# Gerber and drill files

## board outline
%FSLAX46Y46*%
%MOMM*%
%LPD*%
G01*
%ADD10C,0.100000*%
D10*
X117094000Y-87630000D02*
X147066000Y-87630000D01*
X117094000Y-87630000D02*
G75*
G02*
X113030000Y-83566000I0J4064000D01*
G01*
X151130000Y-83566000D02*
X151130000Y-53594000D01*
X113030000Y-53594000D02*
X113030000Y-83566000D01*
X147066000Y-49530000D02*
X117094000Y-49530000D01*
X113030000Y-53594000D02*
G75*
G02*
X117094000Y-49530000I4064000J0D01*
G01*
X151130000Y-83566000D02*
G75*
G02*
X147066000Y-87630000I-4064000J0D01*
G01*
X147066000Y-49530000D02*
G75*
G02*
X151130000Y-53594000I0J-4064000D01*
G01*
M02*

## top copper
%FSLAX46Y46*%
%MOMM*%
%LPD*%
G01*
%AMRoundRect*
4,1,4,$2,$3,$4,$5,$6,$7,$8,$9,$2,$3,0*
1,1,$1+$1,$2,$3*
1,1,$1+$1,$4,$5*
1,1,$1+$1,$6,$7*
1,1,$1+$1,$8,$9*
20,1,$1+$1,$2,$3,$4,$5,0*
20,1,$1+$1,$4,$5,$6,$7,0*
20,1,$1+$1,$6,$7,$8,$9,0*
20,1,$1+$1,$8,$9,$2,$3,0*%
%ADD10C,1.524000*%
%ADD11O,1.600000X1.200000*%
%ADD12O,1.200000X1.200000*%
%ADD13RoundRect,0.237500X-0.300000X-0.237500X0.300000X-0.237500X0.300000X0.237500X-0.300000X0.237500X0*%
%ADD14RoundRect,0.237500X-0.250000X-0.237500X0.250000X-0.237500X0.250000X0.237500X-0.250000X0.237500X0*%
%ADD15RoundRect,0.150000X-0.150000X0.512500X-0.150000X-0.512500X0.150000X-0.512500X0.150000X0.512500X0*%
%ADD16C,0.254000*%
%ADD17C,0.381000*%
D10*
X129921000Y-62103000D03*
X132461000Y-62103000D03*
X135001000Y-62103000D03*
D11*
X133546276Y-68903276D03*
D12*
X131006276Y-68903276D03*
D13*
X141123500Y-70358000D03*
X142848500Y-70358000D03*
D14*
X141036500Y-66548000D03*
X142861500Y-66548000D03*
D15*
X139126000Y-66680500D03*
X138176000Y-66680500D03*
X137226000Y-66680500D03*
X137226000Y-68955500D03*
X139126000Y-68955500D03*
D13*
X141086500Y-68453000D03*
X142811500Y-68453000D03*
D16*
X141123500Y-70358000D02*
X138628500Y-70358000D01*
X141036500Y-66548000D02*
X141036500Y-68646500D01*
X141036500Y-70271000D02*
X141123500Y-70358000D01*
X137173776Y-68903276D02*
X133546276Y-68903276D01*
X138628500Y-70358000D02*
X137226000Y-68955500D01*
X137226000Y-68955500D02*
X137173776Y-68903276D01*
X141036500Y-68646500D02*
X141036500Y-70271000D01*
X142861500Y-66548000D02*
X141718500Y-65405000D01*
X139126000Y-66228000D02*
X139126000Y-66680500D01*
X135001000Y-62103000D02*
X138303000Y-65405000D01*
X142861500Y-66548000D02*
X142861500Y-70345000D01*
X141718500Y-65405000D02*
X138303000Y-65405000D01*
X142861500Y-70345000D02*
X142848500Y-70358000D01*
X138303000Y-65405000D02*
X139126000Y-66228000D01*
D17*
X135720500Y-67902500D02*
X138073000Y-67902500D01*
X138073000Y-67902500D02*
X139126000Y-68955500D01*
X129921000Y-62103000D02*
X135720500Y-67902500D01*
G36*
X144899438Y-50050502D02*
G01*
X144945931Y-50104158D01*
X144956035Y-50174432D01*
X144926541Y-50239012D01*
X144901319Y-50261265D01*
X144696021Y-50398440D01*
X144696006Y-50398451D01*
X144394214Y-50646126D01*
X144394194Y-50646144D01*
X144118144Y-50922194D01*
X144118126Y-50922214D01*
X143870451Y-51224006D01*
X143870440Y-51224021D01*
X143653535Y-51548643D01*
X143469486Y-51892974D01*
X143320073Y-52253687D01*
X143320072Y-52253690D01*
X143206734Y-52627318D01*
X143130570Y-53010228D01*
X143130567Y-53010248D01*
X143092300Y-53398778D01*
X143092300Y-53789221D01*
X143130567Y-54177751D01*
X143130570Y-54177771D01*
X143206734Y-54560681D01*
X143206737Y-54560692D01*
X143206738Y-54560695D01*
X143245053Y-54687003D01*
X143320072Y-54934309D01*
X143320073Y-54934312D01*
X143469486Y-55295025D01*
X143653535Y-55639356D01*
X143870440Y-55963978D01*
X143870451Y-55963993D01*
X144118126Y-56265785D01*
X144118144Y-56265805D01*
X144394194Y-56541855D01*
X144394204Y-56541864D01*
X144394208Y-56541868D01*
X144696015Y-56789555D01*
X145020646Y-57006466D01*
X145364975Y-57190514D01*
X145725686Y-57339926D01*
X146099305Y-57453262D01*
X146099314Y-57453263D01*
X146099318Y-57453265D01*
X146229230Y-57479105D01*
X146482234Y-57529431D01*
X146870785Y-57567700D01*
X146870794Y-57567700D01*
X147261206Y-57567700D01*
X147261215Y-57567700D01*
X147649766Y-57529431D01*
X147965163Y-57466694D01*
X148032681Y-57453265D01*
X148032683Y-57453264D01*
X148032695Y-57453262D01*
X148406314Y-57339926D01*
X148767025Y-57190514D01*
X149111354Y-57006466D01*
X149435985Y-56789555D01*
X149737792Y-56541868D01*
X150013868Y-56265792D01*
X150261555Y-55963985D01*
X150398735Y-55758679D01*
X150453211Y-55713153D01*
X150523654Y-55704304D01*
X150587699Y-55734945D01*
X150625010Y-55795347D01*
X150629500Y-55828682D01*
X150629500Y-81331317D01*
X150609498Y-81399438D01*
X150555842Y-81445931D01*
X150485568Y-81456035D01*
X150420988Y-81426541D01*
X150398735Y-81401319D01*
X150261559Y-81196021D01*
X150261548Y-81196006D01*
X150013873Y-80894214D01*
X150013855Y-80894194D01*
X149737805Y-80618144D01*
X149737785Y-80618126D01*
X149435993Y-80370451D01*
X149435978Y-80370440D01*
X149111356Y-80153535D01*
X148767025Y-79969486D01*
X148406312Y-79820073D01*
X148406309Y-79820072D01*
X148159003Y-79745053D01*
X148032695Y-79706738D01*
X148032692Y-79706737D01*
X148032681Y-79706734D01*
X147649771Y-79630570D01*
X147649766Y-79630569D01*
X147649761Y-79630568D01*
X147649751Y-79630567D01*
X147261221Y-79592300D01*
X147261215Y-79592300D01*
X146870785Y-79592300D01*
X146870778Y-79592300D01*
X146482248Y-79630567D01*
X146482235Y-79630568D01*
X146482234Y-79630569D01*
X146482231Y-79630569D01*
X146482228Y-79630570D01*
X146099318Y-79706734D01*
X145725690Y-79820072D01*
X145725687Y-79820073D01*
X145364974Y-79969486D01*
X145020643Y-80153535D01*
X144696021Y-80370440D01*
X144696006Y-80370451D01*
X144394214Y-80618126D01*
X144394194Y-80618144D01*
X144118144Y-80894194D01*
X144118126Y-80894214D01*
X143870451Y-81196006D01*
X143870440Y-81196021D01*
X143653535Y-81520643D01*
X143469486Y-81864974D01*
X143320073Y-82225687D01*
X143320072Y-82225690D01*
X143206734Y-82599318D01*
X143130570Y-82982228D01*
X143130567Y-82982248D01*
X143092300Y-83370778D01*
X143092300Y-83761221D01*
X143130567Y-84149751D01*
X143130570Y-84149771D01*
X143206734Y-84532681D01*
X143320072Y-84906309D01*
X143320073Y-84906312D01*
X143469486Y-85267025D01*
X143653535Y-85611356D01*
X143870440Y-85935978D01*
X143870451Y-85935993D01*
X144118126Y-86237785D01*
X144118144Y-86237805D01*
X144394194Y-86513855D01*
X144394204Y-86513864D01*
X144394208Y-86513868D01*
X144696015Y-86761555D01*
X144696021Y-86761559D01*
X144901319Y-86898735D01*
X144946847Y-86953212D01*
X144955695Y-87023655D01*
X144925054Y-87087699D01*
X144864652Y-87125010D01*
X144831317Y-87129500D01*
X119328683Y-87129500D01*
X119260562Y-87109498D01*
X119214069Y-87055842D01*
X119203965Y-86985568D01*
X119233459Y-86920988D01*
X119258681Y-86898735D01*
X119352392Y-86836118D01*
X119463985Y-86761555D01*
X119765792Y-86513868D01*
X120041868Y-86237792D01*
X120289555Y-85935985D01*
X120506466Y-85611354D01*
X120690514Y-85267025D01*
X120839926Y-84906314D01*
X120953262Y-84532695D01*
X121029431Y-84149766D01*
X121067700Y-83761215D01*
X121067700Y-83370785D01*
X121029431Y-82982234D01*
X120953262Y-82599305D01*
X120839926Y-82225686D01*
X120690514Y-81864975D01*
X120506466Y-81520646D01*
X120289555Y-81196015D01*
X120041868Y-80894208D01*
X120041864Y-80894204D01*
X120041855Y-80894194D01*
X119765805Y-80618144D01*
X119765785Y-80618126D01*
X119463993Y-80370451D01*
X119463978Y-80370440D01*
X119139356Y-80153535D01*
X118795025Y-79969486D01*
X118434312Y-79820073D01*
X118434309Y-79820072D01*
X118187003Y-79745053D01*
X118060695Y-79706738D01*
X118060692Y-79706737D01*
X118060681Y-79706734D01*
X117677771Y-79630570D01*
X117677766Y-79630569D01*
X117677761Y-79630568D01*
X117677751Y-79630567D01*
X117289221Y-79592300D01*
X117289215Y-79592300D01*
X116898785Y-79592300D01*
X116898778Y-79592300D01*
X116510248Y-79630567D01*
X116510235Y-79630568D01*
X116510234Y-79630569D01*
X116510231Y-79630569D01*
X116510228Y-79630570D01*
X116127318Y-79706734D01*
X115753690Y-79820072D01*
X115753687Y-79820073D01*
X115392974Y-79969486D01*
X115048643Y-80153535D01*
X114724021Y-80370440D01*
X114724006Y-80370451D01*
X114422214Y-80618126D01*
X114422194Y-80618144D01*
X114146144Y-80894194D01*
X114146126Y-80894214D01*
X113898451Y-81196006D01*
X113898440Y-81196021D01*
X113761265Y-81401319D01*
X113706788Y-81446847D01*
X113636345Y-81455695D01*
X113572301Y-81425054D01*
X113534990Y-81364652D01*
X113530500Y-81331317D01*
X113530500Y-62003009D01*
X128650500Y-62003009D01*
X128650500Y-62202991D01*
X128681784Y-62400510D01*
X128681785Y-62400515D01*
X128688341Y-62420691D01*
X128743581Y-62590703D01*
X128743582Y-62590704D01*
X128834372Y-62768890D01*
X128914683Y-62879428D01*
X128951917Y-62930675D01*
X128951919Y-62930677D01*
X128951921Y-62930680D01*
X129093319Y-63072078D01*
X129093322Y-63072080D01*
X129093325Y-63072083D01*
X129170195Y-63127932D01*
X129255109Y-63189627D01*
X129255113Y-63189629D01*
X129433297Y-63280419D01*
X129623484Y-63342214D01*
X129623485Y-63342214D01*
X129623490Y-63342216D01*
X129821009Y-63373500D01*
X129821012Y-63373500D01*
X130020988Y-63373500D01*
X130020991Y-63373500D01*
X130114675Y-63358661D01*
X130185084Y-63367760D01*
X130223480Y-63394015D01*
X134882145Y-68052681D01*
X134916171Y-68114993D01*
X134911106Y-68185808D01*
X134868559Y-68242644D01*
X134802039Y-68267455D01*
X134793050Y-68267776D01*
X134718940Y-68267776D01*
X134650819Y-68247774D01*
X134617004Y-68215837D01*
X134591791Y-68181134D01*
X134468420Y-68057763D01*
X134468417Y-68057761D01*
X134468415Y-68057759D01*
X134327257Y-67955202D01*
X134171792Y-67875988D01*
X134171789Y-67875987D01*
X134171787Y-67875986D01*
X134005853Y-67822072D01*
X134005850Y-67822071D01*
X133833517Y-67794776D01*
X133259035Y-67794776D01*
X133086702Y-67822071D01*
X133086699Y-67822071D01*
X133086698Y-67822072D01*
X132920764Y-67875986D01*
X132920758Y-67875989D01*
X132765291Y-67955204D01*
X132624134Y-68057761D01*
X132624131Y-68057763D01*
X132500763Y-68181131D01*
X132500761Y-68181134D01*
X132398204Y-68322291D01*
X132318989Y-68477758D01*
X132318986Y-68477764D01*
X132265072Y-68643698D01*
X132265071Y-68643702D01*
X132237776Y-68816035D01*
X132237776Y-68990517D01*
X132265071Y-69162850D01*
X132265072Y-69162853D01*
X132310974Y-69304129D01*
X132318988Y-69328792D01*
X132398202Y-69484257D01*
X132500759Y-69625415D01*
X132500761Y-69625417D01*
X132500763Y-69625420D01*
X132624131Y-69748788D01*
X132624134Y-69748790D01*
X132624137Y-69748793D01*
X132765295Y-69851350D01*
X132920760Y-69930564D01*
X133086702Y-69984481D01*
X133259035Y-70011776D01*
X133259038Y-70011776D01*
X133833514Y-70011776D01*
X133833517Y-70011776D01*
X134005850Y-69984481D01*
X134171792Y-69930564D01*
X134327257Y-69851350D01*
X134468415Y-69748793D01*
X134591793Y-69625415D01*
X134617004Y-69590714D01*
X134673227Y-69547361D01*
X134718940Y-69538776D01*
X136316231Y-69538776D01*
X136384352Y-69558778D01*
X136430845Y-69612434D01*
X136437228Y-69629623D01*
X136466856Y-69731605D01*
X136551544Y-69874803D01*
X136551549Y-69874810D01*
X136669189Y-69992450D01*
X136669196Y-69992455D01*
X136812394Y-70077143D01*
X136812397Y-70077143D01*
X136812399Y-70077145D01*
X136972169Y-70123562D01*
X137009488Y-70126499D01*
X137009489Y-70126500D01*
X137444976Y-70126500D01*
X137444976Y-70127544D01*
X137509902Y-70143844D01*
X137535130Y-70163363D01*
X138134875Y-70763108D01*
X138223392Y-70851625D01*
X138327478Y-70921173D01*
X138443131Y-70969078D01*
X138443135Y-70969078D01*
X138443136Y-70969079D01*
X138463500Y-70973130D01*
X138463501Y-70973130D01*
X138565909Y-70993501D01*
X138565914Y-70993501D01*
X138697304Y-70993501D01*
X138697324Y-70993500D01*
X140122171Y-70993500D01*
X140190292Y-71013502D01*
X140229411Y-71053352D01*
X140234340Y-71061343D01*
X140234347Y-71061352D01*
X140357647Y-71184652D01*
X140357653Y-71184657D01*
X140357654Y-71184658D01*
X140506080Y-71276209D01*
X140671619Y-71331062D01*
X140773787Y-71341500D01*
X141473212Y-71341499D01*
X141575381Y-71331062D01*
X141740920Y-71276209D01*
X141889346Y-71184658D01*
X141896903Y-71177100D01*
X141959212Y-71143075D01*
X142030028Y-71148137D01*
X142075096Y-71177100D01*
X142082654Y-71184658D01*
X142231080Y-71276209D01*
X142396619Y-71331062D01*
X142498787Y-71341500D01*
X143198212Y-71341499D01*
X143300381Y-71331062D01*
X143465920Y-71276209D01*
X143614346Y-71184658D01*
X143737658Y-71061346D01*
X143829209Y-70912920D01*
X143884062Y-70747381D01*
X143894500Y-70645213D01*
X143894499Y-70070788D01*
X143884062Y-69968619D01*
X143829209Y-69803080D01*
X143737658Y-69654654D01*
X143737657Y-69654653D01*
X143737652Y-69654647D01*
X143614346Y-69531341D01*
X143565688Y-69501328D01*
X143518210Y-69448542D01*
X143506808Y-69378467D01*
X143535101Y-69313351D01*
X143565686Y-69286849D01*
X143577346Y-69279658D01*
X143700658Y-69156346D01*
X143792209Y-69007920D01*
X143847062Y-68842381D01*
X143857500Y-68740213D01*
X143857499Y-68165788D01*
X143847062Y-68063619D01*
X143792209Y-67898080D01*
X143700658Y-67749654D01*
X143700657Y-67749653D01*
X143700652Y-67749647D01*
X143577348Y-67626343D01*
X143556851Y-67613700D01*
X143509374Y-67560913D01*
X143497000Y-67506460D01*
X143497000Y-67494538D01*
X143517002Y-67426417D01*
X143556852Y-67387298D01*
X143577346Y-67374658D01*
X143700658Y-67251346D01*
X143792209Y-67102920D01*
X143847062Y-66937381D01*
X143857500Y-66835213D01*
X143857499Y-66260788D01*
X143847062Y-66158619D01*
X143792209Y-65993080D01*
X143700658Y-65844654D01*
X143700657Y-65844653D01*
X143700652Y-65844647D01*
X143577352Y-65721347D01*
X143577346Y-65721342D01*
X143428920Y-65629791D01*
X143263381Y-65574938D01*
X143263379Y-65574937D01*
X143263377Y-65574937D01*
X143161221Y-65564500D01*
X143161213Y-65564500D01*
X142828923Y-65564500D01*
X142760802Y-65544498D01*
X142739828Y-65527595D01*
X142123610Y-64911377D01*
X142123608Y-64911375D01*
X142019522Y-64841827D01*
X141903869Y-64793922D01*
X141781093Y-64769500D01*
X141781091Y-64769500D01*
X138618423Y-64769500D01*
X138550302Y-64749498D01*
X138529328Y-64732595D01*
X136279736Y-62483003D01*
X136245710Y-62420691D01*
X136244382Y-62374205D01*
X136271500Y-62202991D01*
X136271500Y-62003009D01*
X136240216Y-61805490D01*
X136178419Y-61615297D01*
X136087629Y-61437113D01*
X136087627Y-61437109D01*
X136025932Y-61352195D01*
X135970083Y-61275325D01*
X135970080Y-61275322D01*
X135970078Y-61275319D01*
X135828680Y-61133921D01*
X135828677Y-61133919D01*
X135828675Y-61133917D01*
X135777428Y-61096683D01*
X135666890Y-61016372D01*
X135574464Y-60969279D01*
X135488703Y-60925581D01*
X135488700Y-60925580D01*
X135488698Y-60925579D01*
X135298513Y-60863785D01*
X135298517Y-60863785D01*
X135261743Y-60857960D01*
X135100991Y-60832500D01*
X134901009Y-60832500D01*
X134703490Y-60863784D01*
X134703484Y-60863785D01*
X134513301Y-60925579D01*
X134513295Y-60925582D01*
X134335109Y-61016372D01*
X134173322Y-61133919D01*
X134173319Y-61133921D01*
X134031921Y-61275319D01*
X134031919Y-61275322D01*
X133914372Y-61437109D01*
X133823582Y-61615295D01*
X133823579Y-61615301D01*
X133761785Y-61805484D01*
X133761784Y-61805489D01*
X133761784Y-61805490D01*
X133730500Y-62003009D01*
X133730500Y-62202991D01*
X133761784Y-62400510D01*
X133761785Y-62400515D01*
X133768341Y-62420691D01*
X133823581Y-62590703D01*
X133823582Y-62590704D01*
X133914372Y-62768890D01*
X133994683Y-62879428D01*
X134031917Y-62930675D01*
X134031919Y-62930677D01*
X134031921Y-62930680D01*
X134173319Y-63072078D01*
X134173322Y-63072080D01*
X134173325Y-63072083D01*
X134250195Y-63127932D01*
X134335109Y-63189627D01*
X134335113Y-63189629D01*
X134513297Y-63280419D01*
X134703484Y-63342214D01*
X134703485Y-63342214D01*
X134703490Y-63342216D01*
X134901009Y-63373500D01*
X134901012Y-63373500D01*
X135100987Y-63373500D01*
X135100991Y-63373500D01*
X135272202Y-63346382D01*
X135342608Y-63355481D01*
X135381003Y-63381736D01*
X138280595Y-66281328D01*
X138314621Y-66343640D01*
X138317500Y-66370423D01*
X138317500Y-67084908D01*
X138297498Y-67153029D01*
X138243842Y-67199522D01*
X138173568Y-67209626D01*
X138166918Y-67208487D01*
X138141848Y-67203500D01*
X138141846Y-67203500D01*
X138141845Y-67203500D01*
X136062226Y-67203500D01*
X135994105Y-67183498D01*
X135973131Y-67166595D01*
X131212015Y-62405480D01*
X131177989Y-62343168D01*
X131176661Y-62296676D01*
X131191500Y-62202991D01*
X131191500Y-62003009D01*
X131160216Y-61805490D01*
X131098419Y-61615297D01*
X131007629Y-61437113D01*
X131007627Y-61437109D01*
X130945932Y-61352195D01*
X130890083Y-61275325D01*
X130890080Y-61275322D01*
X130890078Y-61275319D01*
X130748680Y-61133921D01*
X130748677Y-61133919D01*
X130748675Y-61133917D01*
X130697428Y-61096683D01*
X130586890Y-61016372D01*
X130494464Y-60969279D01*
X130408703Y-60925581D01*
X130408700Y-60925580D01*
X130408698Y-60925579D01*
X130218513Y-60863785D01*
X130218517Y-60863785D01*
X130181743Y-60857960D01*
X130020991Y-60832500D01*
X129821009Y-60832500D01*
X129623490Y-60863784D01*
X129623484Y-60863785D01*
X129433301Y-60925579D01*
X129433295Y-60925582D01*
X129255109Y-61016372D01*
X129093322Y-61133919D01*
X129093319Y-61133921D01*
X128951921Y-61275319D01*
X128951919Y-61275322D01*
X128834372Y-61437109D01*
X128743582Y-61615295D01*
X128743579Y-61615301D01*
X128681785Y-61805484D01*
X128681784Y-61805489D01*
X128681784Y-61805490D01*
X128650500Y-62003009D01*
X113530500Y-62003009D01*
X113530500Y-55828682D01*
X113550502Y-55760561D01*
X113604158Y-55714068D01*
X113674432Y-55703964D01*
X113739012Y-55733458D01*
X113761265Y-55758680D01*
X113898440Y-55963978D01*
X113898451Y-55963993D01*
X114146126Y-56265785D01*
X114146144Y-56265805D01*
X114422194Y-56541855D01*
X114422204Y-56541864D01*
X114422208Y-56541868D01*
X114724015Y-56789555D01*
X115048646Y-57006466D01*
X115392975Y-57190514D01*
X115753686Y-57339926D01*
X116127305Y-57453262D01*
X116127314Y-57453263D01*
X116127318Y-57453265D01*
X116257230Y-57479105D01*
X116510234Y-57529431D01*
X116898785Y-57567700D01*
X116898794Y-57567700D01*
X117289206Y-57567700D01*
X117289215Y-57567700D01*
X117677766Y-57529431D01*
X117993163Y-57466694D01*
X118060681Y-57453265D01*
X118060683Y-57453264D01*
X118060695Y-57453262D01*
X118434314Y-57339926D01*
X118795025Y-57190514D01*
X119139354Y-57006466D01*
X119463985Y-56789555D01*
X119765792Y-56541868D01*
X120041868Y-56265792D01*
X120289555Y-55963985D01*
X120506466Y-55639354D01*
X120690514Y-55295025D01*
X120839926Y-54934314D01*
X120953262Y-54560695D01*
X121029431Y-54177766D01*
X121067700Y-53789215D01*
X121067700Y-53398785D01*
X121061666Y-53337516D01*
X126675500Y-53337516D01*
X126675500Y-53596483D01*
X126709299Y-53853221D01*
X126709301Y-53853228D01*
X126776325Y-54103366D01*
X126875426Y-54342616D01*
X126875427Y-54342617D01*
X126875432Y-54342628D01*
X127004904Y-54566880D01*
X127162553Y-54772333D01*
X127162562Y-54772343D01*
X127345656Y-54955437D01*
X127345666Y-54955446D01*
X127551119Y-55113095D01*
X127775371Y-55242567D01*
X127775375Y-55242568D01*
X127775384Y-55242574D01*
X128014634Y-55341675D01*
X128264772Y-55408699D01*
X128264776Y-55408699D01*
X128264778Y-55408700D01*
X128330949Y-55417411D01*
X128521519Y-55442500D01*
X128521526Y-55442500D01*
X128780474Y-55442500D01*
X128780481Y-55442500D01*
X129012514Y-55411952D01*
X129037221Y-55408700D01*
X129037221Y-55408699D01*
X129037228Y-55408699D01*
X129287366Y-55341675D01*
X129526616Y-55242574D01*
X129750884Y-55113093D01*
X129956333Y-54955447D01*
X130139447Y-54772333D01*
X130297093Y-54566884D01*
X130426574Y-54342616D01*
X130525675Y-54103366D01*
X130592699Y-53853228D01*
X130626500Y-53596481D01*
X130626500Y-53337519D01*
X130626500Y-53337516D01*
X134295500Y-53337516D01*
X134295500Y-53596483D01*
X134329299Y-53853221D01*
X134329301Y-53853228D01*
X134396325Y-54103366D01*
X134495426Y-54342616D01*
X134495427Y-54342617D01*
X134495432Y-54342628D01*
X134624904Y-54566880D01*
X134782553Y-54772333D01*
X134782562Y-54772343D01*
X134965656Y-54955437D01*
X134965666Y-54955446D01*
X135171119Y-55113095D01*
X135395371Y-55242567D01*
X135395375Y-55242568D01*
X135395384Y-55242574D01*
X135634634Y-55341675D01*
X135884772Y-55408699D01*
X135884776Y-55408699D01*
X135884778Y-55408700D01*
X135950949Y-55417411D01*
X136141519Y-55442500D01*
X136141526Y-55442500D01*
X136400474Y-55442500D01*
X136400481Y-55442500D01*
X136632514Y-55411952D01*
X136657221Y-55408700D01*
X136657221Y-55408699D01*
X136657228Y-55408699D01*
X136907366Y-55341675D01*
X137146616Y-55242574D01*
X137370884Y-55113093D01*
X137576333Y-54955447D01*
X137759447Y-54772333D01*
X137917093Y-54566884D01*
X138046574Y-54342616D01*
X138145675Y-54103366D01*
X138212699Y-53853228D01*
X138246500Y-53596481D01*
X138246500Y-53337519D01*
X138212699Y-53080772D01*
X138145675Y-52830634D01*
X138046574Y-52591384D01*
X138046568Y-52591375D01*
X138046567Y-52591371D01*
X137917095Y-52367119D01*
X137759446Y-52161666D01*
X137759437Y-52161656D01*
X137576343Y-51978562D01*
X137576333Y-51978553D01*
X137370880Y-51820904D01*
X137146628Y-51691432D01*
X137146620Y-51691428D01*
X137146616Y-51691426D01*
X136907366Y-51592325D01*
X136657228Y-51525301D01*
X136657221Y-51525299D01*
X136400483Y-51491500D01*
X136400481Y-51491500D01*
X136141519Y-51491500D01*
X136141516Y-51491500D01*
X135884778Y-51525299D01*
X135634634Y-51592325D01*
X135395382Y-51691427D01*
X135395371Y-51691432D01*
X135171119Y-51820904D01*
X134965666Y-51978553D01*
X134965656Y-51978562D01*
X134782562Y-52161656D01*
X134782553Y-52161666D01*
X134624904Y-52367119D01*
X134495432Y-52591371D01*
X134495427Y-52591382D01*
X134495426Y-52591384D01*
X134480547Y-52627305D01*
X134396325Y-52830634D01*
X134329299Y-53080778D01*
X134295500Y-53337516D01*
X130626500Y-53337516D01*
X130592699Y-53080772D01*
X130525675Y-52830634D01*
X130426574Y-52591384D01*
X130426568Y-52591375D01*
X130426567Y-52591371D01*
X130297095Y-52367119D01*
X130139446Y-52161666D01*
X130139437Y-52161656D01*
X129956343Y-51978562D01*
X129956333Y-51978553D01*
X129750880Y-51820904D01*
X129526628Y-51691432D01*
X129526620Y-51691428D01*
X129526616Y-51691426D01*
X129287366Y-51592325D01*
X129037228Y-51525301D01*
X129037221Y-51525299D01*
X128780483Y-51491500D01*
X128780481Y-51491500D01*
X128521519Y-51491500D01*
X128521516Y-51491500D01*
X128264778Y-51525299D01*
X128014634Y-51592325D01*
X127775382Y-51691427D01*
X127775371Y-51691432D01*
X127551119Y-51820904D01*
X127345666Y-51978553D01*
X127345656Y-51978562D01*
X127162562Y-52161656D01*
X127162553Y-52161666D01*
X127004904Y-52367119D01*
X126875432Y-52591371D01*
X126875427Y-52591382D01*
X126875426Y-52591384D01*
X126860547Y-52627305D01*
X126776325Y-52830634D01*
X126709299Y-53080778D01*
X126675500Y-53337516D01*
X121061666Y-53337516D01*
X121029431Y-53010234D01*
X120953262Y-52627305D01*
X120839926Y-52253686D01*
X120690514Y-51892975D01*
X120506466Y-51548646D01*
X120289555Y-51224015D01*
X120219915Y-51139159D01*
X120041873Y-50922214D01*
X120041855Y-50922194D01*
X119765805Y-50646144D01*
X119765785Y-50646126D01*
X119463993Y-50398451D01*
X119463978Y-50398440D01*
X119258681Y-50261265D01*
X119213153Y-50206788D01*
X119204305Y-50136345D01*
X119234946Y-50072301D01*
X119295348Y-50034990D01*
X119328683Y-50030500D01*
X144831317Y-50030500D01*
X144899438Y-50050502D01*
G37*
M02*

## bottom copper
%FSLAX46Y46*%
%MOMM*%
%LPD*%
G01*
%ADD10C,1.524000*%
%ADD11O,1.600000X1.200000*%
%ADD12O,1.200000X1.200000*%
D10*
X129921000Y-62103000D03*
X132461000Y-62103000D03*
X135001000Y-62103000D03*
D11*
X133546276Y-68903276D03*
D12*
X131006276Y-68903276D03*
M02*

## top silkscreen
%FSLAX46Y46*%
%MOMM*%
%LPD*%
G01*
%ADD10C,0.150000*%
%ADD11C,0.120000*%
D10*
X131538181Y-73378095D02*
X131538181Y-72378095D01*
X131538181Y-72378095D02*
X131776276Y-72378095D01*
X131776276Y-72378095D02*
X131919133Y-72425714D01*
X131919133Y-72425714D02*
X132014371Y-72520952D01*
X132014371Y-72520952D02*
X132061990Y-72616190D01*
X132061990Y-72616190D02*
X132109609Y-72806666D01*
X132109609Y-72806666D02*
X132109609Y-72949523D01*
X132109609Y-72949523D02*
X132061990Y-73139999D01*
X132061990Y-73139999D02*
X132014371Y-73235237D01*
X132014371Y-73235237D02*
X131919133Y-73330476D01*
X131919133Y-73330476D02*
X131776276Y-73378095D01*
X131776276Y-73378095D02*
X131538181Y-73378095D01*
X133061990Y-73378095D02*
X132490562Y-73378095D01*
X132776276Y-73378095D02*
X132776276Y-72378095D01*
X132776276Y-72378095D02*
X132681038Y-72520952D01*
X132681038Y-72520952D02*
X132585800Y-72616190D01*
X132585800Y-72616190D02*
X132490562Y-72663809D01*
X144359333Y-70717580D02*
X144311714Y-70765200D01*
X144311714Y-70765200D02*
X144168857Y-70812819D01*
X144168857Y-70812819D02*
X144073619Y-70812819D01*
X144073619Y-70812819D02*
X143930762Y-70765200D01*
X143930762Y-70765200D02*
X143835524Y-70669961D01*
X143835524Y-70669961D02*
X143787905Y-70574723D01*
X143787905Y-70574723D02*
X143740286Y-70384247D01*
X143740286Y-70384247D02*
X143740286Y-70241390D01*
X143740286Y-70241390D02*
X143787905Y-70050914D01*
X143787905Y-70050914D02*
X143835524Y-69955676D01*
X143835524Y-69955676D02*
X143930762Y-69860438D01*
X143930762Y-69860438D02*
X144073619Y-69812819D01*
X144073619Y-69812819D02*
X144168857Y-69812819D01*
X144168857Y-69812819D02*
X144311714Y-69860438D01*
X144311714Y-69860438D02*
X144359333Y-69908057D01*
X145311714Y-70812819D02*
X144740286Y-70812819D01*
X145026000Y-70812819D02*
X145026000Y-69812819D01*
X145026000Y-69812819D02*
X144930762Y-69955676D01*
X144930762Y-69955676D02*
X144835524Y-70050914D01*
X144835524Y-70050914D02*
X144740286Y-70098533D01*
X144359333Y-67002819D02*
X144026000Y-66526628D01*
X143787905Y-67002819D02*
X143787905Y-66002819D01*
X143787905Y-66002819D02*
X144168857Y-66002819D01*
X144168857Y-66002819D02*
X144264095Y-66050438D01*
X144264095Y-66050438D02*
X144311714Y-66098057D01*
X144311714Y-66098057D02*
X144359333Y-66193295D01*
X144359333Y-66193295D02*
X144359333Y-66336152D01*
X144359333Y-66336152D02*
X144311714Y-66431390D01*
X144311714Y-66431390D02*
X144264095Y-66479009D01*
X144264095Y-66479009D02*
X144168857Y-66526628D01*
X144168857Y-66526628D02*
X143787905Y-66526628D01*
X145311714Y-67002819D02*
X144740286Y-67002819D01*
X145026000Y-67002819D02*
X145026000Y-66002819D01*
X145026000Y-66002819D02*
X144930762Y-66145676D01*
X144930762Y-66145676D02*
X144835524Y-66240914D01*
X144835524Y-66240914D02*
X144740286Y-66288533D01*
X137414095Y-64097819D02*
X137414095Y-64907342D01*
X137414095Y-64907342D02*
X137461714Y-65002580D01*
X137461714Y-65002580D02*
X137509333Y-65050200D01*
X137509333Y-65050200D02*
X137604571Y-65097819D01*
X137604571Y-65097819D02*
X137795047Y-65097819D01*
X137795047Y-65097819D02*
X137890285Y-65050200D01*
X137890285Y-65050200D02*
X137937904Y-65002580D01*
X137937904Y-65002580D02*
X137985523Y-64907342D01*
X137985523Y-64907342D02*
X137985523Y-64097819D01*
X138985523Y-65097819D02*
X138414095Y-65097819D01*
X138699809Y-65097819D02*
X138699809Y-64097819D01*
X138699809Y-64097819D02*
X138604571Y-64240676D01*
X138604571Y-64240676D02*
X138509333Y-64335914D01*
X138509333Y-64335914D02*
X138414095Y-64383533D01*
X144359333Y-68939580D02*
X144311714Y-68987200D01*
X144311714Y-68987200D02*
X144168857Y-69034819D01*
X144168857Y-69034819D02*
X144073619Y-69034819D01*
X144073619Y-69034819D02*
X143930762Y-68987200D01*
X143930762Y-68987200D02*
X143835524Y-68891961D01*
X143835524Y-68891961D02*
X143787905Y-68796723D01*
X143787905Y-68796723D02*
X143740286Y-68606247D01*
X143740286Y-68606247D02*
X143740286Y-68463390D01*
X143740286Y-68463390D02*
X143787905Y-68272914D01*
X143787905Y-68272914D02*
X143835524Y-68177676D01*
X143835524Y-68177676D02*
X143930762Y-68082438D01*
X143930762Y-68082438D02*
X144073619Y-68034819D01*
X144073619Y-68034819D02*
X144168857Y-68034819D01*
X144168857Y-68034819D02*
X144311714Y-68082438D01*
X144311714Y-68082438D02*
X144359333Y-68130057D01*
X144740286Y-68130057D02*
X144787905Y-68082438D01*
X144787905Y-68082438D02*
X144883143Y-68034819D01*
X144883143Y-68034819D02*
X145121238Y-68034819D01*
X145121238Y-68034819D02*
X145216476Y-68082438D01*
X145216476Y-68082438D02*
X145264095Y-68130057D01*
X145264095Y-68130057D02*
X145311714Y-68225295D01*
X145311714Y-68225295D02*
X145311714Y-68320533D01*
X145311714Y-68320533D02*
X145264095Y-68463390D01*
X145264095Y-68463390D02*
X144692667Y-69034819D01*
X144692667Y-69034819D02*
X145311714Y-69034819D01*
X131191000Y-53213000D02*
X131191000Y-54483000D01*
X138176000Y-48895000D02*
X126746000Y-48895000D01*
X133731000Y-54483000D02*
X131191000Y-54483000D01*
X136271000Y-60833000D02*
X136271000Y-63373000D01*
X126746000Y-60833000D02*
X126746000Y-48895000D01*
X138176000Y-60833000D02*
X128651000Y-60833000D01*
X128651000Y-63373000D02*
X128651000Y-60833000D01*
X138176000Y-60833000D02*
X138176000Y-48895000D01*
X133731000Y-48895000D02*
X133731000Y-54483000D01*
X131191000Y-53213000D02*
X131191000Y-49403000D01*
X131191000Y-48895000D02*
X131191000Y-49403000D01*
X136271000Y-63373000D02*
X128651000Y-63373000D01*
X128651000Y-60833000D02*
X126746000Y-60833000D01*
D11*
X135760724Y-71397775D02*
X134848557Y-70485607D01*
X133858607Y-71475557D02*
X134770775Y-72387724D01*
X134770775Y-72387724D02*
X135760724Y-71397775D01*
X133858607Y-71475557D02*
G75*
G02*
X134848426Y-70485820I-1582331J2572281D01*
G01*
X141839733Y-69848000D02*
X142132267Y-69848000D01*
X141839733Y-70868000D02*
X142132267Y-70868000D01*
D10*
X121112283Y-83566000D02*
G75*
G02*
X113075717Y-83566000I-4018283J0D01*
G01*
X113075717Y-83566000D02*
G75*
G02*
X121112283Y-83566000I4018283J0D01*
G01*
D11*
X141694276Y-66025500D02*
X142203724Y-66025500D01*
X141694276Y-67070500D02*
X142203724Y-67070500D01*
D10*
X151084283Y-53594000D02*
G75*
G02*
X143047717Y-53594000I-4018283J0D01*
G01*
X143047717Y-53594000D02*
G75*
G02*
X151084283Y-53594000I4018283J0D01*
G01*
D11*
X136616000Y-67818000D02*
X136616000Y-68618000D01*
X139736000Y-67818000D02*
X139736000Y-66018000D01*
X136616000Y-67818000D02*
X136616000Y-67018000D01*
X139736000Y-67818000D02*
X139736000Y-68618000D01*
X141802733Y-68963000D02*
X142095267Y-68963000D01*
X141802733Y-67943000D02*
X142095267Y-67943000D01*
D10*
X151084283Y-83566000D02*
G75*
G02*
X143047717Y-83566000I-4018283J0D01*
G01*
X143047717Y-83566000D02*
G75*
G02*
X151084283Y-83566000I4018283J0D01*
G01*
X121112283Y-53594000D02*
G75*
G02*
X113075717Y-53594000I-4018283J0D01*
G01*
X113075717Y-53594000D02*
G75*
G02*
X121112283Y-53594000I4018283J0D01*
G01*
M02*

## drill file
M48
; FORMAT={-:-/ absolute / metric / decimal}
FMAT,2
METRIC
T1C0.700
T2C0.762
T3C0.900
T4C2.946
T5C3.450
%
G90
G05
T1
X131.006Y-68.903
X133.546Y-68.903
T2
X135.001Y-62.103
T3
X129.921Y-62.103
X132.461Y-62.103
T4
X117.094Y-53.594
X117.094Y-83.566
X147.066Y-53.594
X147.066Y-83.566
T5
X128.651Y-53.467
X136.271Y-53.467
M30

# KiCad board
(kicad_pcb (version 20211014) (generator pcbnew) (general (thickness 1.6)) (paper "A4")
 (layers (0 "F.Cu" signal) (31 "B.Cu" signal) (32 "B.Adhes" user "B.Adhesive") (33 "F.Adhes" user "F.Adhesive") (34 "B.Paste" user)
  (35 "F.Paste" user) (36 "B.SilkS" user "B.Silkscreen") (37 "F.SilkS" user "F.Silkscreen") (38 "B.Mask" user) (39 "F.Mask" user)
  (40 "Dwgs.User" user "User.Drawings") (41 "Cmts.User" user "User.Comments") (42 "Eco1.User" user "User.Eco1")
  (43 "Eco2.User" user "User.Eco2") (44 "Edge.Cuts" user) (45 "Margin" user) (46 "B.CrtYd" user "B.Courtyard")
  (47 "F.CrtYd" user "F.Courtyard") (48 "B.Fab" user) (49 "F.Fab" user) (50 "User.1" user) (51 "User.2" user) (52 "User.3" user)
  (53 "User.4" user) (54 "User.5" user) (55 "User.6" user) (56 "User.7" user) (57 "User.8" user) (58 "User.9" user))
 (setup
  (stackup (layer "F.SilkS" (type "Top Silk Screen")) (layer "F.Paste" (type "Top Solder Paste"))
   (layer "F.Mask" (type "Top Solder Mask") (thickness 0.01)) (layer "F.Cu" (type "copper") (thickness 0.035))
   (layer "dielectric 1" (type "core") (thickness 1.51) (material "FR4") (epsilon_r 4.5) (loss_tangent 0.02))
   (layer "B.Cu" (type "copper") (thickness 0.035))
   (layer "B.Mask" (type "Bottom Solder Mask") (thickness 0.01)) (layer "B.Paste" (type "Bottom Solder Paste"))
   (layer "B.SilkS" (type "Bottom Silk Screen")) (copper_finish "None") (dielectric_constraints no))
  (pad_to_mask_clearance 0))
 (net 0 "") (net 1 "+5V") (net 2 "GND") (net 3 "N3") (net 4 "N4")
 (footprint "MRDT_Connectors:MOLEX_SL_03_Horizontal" (layer "F.Cu") (at 129.921 62.103)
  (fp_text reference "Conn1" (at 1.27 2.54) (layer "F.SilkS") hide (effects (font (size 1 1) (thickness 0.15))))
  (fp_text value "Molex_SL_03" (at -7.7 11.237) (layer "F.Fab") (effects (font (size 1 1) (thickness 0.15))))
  (fp_line (start 1.27 -8.89) (end 1.27 -7.62) (layer "F.SilkS") (width 0.15))
  (fp_line (start 8.255 -13.208) (end -3.175 -13.208) (layer "F.SilkS") (width 0.15))
  (fp_line (start 3.81 -7.62) (end 1.27 -7.62) (layer "F.SilkS") (width 0.15))
  (fp_line (start 6.35 -1.27) (end 6.35 1.27) (layer "F.SilkS") (width 0.15))
  (fp_line (start -3.175 -1.27) (end -3.175 -13.208) (layer "F.SilkS") (width 0.15))
  (fp_line (start 8.255 -1.27) (end -1.27 -1.27) (layer "F.SilkS") (width 0.15))
  (fp_line (start -1.27 1.27) (end -1.27 -1.27) (layer "F.SilkS") (width 0.15))
  (fp_line (start 8.255 -1.27) (end 8.255 -13.208) (layer "F.SilkS") (width 0.15))
  (fp_line (start 3.81 -13.208) (end 3.81 -7.62) (layer "F.SilkS") (width 0.15))
  (fp_line (start 1.27 -8.89) (end 1.27 -12.7) (layer "F.SilkS") (width 0.15))
  (fp_line (start 1.27 -13.208) (end 1.27 -12.7) (layer "F.SilkS") (width 0.15))
  (fp_line (start 6.35 1.27) (end -1.27 1.27) (layer "F.SilkS") (width 0.15))
  (fp_line (start -1.27 -1.27) (end -3.175 -1.27) (layer "F.SilkS") (width 0.15))
  (pad "" np_thru_hole circle locked (at 6.35 -8.636) (size 3.45 3.45) (drill 3.45) (layers *.Cu *.Mask))
  (pad "" np_thru_hole circle locked (at -1.27 -8.636) (size 3.45 3.45) (drill 3.45) (layers *.Cu *.Mask))
  (pad "1" thru_hole circle locked (at 0 0) (size 1.524 1.524) (drill 0.9) (layers *.Cu *.Mask) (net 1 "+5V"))
  (pad "2" thru_hole circle locked (at 2.54 0) (size 1.524 1.524) (drill 0.9) (layers *.Cu *.Mask) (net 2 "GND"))
  (pad "3" thru_hole circle locked (at 5.08 0) (size 1.524 1.524) (drill 0.762) (layers *.Cu *.Mask) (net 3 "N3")))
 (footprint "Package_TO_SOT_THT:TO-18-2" (layer "F.Cu") (at 133.546276 68.903276 180)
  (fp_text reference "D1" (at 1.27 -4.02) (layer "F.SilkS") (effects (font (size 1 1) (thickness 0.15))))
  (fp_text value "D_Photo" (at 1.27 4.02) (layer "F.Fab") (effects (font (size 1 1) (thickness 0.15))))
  (fp_line (start -2.214448 -2.494499) (end -1.302281 -1.582331) (layer "F.SilkS") (width 0.12))
  (fp_line (start -0.312331 -2.572281) (end -1.224499 -3.484448) (layer "F.SilkS") (width 0.12))
  (fp_line (start -1.224499 -3.484448) (end -2.214448 -2.494499) (layer "F.SilkS") (width 0.12))
  (fp_arc (start -0.312331 -2.572281) (mid 3.405374 2.135551) (end -1.30215 -1.582544) (layer "F.SilkS") (width 0.12))
  (pad "1" thru_hole oval (at 0 0 180) (size 1.6 1.2) (drill 0.7) (layers *.Cu *.Mask) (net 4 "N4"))
  (pad "2" thru_hole oval (at 2.54 0 180) (size 1.2 1.2) (drill 0.7) (layers *.Cu *.Mask) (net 2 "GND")))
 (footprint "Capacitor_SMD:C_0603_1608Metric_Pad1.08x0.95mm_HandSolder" (layer "F.Cu") (at 141.986 70.358)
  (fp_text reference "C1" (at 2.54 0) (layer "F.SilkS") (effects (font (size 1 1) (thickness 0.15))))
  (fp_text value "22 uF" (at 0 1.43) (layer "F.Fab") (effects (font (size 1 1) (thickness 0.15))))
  (fp_line (start -0.146267 -0.51) (end 0.146267 -0.51) (layer "F.SilkS") (width 0.12))
  (fp_line (start -0.146267 0.51) (end 0.146267 0.51) (layer "F.SilkS") (width 0.12))
  (pad "1" smd roundrect (at -0.8625 0) (size 1.075 0.95) (layers "F.Cu" "F.Paste" "F.Mask") (roundrect_rratio 0.25) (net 4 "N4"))
  (pad "2" smd roundrect (at 0.8625 0) (size 1.075 0.95) (layers "F.Cu" "F.Paste" "F.Mask") (roundrect_rratio 0.25) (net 3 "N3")))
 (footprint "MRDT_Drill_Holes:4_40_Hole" (layer "F.Cu") (at 117.094 83.566) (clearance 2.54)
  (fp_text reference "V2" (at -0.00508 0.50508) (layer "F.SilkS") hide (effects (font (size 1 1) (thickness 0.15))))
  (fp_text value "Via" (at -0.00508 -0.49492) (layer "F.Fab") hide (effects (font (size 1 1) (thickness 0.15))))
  (fp_circle (center 0 0) (end -0.00508 4.01828) (layer "F.SilkS") (width 0.15) (fill none))
  (pad "" np_thru_hole circle locked (at 0 0) (size 2.9464 2.9464) (drill 2.9464) (layers *.Cu *.Mask) (clearance 2.5)))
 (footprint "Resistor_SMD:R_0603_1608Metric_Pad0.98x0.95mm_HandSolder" (layer "F.Cu") (at 141.949 66.548)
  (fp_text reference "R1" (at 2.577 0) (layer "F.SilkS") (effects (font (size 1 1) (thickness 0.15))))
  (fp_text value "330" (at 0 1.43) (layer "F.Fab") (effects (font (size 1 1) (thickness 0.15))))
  (fp_line (start -0.254724 -0.5225) (end 0.254724 -0.5225) (layer "F.SilkS") (width 0.12))
  (fp_line (start -0.254724 0.5225) (end 0.254724 0.5225) (layer "F.SilkS") (width 0.12))
  (pad "1" smd roundrect (at -0.9125 0) (size 0.975 0.95) (layers "F.Cu" "F.Paste" "F.Mask") (roundrect_rratio 0.25) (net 4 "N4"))
  (pad "2" smd roundrect (at 0.9125 0) (size 0.975 0.95) (layers "F.Cu" "F.Paste" "F.Mask") (roundrect_rratio 0.25) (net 3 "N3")))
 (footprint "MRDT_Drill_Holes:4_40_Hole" (layer "F.Cu") (at 147.066 53.594) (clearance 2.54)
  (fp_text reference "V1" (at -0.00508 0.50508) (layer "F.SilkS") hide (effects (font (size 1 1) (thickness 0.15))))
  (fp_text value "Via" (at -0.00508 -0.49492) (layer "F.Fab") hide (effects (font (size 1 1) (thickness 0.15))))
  (fp_circle (center 0 0) (end -0.00508 4.01828) (layer "F.SilkS") (width 0.15) (fill none))
  (pad "" np_thru_hole circle locked (at 0 0) (size 2.9464 2.9464) (drill 2.9464) (layers *.Cu *.Mask) (clearance 2.5)))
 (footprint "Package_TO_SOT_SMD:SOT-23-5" (layer "F.Cu") (at 138.176 67.818 -90)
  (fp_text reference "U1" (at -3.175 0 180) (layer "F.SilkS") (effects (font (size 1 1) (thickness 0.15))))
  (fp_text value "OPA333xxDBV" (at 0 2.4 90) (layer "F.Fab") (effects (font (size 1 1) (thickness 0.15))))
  (fp_line (start 0 1.56) (end 0.8 1.56) (layer "F.SilkS") (width 0.12))
  (fp_line (start 0 -1.56) (end -1.8 -1.56) (layer "F.SilkS") (width 0.12))
  (fp_line (start 0 1.56) (end -0.8 1.56) (layer "F.SilkS") (width 0.12))
  (fp_line (start 0 -1.56) (end 0.8 -1.56) (layer "F.SilkS") (width 0.12))
  (pad "1" smd roundrect (at -1.1375 -0.95 270) (size 1.325 0.6) (layers "F.Cu" "F.Paste" "F.Mask") (roundrect_rratio 0.25) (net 3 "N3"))
  (pad "2" smd roundrect (at -1.1375 0 270) (size 1.325 0.6) (layers "F.Cu" "F.Paste" "F.Mask") (roundrect_rratio 0.25) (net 2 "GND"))
  (pad "3" smd roundrect (at -1.1375 0.95 270) (size 1.325 0.6) (layers "F.Cu" "F.Paste" "F.Mask") (roundrect_rratio 0.25) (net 2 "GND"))
  (pad "4" smd roundrect (at 1.1375 0.95 270) (size 1.325 0.6) (layers "F.Cu" "F.Paste" "F.Mask") (roundrect_rratio 0.25) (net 4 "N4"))
  (pad "5" smd roundrect (at 1.1375 -0.95 270) (size 1.325 0.6) (layers "F.Cu" "F.Paste" "F.Mask") (roundrect_rratio 0.25) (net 1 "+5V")))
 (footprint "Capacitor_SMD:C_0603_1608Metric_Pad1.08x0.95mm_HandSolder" (layer "F.Cu") (at 141.949 68.453)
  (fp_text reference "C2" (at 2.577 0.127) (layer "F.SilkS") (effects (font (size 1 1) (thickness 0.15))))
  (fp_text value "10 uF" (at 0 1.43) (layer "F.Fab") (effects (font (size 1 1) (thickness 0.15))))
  (fp_line (start -0.146267 0.51) (end 0.146267 0.51) (layer "F.SilkS") (width 0.12))
  (fp_line (start -0.146267 -0.51) (end 0.146267 -0.51) (layer "F.SilkS") (width 0.12))
  (pad "1" smd roundrect (at -0.8625 0) (size 1.075 0.95) (layers "F.Cu" "F.Paste" "F.Mask") (roundrect_rratio 0.25) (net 4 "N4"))
  (pad "2" smd roundrect (at 0.8625 0) (size 1.075 0.95) (layers "F.Cu" "F.Paste" "F.Mask") (roundrect_rratio 0.25) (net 3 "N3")))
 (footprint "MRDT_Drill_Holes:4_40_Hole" (layer "F.Cu") (at 147.066 83.566) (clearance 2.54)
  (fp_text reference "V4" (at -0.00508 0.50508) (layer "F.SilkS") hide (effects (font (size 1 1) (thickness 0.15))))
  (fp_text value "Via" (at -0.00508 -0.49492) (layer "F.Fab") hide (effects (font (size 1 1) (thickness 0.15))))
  (fp_circle (center 0 0) (end -0.00508 4.01828) (layer "F.SilkS") (width 0.15) (fill none))
  (pad "" np_thru_hole circle locked (at 0 0) (size 2.9464 2.9464) (drill 2.9464) (layers *.Cu *.Mask) (clearance 2.5)))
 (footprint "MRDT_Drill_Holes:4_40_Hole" (layer "F.Cu") (at 117.094 53.594) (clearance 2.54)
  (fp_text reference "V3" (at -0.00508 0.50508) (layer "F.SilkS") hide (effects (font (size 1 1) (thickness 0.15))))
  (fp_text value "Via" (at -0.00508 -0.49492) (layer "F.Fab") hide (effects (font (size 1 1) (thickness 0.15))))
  (fp_circle (center 0 0) (end -0.00508 4.01828) (layer "F.SilkS") (width 0.15) (fill none))
  (pad "" np_thru_hole circle locked (at 0 0) (size 2.9464 2.9464) (drill 2.9464) (layers *.Cu *.Mask) (clearance 2.5)))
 (gr_line (start 117.094 87.63) (end 147.066 87.63) (layer "Edge.Cuts") (width 0.1))
 (gr_arc (start 117.094 87.63) (mid 114.220318 86.439682) (end 113.03 83.566) (layer "Edge.Cuts") (width 0.1))
 (gr_line (start 151.13 83.566) (end 151.13 53.594) (layer "Edge.Cuts") (width 0.1))
 (gr_line (start 113.03 53.594) (end 113.03 83.566) (layer "Edge.Cuts") (width 0.1))
 (gr_line (start 147.066 49.53) (end 117.094 49.53) (layer "Edge.Cuts") (width 0.1))
 (gr_arc (start 113.03 53.594) (mid 114.220318 50.720318) (end 117.094 49.53) (layer "Edge.Cuts") (width 0.1))
 (gr_arc (start 151.13 83.566) (mid 149.939682 86.439682) (end 147.066 87.63) (layer "Edge.Cuts") (width 0.1))
 (gr_arc (start 147.066 49.53) (mid 149.939682 50.720318) (end 151.13 53.594) (layer "Edge.Cuts") (width 0.1))
 (segment (start 141.1235 70.358) (end 138.6285 70.358) (width 0.254) (layer "F.Cu") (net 4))
 (segment (start 141.0365 66.548) (end 141.0365 68.6465) (width 0.254) (layer "F.Cu") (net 4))
 (segment (start 141.0365 70.271) (end 141.1235 70.358) (width 0.254) (layer "F.Cu") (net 4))
 (segment (start 137.173776 68.903276) (end 133.546276 68.903276) (width 0.254) (layer "F.Cu") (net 4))
 (segment (start 138.6285 70.358) (end 137.226 68.9555) (width 0.254) (layer "F.Cu") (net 4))
 (segment (start 137.226 68.9555) (end 137.173776 68.903276) (width 0.254) (layer "F.Cu") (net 4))
 (segment (start 141.0365 68.6465) (end 141.0365 70.271) (width 0.254) (layer "F.Cu") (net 4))
 (segment (start 142.8615 66.548) (end 141.7185 65.405) (width 0.254) (layer "F.Cu") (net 3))
 (segment (start 139.126 66.228) (end 139.126 66.6805) (width 0.254) (layer "F.Cu") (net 3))
 (segment (start 135.001 62.103) (end 138.303 65.405) (width 0.254) (layer "F.Cu") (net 3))
 (segment (start 142.8615 66.548) (end 142.8615 70.345) (width 0.254) (layer "F.Cu") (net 3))
 (segment (start 141.7185 65.405) (end 138.303 65.405) (width 0.254) (layer "F.Cu") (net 3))
 (segment (start 142.8615 70.345) (end 142.8485 70.358) (width 0.254) (layer "F.Cu") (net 3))
 (segment (start 138.303 65.405) (end 139.126 66.228) (width 0.254) (layer "F.Cu") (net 3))
 (segment (start 135.7205 67.9025) (end 138.073 67.9025) (width 0.381) (layer "F.Cu") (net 1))
 (segment (start 138.073 67.9025) (end 139.126 68.9555) (width 0.381) (layer "F.Cu") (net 1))
 (segment (start 129.921 62.103) (end 135.7205 67.9025) (width 0.381) (layer "F.Cu") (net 1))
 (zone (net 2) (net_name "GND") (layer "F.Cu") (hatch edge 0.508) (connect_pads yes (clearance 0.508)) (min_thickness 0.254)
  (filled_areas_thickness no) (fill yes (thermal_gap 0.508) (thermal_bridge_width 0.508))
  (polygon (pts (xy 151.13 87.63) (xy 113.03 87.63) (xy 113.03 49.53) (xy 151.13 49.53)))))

